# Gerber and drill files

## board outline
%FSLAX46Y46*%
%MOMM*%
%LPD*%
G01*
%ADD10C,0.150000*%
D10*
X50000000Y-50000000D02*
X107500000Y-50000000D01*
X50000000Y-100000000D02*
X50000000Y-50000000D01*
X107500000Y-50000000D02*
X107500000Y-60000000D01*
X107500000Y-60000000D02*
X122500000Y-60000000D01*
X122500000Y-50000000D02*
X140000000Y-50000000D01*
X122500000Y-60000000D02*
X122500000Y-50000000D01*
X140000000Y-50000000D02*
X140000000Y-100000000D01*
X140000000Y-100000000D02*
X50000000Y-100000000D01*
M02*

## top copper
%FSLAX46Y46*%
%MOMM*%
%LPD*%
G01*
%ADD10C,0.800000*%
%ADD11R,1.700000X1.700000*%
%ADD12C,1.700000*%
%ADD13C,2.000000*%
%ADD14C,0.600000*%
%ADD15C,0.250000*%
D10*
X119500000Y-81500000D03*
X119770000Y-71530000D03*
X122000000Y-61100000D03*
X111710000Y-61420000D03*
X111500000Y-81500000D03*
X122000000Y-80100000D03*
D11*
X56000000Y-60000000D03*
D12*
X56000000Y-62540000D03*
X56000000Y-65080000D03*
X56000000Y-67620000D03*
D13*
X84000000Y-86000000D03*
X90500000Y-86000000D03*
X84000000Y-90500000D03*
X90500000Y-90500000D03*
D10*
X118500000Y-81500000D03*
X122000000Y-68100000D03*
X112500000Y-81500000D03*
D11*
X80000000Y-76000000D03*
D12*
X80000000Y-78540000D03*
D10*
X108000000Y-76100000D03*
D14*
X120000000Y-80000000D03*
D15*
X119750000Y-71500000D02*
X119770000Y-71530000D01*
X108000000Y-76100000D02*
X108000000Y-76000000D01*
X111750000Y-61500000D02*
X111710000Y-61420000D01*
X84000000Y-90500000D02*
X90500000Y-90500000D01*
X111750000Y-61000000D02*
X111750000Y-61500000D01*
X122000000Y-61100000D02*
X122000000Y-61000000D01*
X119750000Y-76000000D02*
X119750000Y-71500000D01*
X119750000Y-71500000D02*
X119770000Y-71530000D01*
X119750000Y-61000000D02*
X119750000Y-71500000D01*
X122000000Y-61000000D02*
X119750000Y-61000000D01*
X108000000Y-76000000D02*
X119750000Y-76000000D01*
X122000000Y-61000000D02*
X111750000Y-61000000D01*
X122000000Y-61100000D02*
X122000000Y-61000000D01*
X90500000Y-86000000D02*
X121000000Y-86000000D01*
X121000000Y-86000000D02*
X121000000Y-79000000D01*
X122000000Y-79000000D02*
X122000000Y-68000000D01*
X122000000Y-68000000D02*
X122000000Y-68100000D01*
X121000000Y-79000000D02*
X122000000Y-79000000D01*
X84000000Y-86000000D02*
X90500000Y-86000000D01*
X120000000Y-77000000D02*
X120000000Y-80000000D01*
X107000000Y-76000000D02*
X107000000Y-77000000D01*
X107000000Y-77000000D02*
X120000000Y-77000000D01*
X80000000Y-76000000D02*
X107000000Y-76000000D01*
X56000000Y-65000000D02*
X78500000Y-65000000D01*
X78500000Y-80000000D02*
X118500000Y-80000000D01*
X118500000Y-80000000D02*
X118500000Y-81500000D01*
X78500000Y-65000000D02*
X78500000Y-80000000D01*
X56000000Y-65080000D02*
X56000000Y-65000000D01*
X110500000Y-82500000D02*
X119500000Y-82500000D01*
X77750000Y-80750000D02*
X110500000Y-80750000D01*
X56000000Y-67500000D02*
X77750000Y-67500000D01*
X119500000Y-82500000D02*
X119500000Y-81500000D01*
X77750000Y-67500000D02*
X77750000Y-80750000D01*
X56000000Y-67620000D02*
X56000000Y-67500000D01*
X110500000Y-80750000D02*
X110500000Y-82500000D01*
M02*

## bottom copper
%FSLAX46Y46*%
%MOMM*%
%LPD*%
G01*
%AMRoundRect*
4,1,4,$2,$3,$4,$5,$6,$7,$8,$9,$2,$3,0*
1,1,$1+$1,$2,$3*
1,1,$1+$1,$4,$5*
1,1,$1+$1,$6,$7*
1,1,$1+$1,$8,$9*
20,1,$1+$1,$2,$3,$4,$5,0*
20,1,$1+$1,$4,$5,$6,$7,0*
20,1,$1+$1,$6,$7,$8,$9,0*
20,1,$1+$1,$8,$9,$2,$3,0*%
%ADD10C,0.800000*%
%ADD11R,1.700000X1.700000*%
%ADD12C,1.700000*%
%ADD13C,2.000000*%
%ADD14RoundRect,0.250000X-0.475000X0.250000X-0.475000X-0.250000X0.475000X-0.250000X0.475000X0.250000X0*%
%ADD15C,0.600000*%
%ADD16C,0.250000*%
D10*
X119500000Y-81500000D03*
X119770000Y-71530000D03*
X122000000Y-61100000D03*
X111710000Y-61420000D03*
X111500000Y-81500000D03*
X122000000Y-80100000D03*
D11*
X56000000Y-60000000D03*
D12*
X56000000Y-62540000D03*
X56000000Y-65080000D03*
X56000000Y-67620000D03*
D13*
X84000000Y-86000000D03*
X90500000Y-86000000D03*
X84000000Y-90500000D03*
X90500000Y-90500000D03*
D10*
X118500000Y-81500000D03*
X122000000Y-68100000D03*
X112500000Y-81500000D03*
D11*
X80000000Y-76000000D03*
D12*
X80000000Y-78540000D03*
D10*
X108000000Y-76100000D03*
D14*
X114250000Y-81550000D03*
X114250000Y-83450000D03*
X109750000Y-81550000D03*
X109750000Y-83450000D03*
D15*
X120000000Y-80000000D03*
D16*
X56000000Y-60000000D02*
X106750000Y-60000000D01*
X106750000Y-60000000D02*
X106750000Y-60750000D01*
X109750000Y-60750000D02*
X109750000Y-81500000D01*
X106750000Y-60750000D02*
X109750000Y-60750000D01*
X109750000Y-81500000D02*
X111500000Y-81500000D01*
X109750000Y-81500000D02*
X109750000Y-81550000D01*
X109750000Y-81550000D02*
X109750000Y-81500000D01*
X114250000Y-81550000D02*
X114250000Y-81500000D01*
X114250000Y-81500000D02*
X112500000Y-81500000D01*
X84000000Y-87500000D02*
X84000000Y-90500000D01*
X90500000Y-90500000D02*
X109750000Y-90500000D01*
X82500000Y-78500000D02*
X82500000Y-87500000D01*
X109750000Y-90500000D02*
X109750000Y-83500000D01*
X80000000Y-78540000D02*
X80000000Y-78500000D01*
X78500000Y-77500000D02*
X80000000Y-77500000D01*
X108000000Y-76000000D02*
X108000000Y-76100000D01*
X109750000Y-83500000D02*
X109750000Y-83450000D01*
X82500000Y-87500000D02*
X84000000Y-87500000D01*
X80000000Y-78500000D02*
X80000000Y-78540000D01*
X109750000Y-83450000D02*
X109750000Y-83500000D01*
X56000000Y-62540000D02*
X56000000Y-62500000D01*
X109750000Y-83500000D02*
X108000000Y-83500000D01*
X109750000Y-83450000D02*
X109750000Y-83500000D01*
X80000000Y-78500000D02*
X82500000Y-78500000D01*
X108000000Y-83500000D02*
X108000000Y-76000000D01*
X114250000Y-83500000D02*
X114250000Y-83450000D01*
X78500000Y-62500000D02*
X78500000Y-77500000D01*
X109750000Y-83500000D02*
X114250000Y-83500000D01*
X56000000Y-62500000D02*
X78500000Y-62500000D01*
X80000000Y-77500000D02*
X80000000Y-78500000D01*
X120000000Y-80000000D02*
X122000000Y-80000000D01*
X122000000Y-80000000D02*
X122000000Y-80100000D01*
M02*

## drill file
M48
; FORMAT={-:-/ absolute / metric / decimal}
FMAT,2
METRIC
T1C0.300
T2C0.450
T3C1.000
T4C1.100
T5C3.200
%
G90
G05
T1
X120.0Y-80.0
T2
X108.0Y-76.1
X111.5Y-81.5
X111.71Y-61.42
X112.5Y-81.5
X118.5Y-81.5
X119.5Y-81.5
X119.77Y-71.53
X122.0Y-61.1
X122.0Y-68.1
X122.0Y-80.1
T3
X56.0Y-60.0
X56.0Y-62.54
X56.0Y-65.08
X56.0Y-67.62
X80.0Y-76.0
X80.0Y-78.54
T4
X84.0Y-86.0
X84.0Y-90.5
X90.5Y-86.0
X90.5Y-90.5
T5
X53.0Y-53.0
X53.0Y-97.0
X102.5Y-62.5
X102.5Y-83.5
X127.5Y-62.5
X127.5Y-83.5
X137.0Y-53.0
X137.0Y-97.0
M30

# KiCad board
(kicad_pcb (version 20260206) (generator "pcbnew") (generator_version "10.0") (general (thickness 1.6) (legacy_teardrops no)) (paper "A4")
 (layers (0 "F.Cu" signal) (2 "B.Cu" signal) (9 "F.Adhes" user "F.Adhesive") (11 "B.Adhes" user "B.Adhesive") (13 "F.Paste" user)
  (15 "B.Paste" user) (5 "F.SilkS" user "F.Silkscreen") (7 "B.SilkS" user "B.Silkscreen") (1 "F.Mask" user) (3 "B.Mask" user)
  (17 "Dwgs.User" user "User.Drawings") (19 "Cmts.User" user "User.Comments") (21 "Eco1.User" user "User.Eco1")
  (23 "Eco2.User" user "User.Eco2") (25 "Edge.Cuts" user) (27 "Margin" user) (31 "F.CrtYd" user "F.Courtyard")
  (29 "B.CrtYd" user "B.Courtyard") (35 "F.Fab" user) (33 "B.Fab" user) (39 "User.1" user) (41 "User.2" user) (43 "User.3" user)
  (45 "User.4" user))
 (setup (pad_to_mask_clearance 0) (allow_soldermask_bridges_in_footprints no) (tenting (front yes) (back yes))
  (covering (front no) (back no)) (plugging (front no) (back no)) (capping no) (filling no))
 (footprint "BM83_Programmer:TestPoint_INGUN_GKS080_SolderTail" (layer "F.Cu") (at 119.5 81.5)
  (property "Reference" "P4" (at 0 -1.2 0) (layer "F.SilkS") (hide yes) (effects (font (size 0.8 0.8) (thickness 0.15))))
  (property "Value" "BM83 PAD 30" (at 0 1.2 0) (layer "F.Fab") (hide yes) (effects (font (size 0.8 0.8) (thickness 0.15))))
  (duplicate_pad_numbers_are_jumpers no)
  (pad "1" thru_hole circle (at 0 0) (size 0.8 0.8) (drill 0.45) (layers "*.Cu" "*.Mask") (remove_unused_layers no) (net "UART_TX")))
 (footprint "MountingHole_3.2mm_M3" (layer "F.Cu") (at 53 97)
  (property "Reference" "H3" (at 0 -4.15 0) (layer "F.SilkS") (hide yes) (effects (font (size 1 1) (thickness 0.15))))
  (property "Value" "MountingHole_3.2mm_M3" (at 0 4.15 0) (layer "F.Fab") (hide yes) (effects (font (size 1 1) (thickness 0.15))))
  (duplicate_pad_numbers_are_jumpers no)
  (pad "" np_thru_hole circle (at 0 0) (size 3.2 3.2) (drill 3.2) (layers "*.Cu" "*.Mask")))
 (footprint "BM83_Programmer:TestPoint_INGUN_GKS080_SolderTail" (layer "F.Cu") (at 119.77 71.53)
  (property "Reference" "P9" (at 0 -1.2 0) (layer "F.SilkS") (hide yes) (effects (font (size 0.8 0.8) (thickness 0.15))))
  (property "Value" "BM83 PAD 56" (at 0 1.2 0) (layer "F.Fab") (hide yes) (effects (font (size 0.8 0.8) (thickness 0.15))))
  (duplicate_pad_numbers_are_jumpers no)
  (pad "1" thru_hole circle (at 0 0) (size 0.8 0.8) (drill 0.45) (layers "*.Cu" "*.Mask") (remove_unused_layers no) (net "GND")))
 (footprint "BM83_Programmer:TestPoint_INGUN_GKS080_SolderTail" (layer "F.Cu") (at 122 61.1)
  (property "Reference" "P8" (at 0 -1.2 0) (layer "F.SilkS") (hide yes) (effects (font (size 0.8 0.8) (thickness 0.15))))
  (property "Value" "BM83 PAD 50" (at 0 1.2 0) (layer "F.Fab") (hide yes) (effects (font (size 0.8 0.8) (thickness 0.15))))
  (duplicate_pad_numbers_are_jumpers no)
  (pad "1" thru_hole circle (at 0 0) (size 0.8 0.8) (drill 0.45) (layers "*.Cu" "*.Mask") (remove_unused_layers no) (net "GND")))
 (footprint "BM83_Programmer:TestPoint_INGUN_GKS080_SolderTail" (layer "F.Cu") (at 111.71 61.42)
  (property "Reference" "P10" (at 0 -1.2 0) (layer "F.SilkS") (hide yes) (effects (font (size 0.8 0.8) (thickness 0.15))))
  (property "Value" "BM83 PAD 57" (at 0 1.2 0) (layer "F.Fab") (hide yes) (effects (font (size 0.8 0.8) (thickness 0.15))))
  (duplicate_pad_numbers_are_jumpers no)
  (pad "1" thru_hole circle (at 0 0) (size 0.8 0.8) (drill 0.45) (layers "*.Cu" "*.Mask") (remove_unused_layers no) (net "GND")))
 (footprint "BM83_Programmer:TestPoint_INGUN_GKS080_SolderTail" (layer "F.Cu") (at 111.5 81.5)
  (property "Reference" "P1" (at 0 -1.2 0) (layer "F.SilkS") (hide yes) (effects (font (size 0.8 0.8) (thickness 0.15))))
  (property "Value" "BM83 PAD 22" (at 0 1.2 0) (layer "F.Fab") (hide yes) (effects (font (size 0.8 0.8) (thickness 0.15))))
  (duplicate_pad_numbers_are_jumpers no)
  (pad "1" thru_hole circle (at 0 0) (size 0.8 0.8) (drill 0.45) (layers "*.Cu" "*.Mask") (remove_unused_layers no) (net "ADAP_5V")))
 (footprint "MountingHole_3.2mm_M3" (layer "F.Cu") (at 102.5 62.5)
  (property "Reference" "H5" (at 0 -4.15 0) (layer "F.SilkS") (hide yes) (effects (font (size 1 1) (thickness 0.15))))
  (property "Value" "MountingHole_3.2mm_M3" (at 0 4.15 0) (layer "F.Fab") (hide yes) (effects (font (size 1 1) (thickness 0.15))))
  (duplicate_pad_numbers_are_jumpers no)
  (pad "" np_thru_hole circle (at 0 0) (size 3.2 3.2) (drill 3.2) (layers "*.Cu" "*.Mask")))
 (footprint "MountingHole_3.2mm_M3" (layer "F.Cu") (at 127.5 83.5)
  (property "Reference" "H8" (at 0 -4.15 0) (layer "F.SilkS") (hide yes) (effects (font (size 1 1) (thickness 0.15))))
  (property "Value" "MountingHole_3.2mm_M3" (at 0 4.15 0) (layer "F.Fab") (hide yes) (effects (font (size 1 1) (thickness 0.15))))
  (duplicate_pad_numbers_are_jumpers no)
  (pad "" np_thru_hole circle (at 0 0) (size 3.2 3.2) (drill 3.2) (layers "*.Cu" "*.Mask")))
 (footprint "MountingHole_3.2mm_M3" (layer "F.Cu") (at 53 53)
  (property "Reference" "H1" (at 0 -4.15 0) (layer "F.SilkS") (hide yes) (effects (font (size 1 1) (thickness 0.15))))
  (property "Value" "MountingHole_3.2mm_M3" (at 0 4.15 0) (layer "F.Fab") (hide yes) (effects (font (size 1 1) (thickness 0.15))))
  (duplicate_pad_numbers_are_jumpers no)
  (pad "" np_thru_hole circle (at 0 0) (size 3.2 3.2) (drill 3.2) (layers "*.Cu" "*.Mask")))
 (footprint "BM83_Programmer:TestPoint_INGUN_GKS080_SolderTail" (layer "F.Cu") (at 122 80.1)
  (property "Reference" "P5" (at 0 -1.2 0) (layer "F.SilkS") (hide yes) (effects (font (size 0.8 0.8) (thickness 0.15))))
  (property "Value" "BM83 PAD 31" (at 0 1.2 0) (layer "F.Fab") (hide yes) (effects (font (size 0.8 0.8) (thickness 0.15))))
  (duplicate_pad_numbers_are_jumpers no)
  (pad "1" thru_hole circle (at 0 0) (size 0.8 0.8) (drill 0.45) (layers "*.Cu" "*.Mask") (remove_unused_layers no) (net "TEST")))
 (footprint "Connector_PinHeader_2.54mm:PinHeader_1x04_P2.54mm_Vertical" (layer "F.Cu") (at 56 60)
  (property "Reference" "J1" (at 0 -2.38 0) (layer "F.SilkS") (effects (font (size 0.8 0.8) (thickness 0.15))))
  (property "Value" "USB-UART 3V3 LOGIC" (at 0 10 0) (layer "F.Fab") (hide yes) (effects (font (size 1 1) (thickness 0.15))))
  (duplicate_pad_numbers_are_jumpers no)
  (pad "1" thru_hole rect (at 0 0) (size 1.7 1.7) (drill 1) (layers "*.Cu" "*.Mask") (remove_unused_layers no) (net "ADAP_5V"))
  (pad "2" thru_hole circle (at 0 2.54) (size 1.7 1.7) (drill 1) (layers "*.Cu" "*.Mask") (remove_unused_layers no) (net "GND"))
  (pad "3" thru_hole circle (at 0 5.08) (size 1.7 1.7) (drill 1) (layers "*.Cu" "*.Mask") (remove_unused_layers no) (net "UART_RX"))
  (pad "4" thru_hole circle (at 0 7.62) (size 1.7 1.7) (drill 1) (layers "*.Cu" "*.Mask") (remove_unused_layers no) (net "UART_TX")))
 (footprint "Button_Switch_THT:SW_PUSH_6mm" (layer "F.Cu") (at 84 86)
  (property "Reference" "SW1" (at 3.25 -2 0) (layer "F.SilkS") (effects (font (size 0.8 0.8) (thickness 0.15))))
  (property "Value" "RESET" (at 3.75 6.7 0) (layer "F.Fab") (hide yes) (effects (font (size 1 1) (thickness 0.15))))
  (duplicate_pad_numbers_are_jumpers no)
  (pad "1" thru_hole circle (at 0 0 90) (size 2 2) (drill 1.1) (layers "*.Cu" "*.Mask") (remove_unused_layers no) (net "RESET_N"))
  (pad "1" thru_hole circle (at 6.5 0 90) (size 2 2) (drill 1.1) (layers "*.Cu" "*.Mask") (remove_unused_layers no) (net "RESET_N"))
  (pad "2" thru_hole circle (at 0 4.5 90) (size 2 2) (drill 1.1) (layers "*.Cu" "*.Mask") (remove_unused_layers no) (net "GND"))
  (pad "2" thru_hole circle (at 6.5 4.5 90) (size 2 2) (drill 1.1) (layers "*.Cu" "*.Mask") (remove_unused_layers no) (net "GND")))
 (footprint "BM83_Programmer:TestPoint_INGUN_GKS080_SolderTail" (layer "F.Cu") (at 118.5 81.5)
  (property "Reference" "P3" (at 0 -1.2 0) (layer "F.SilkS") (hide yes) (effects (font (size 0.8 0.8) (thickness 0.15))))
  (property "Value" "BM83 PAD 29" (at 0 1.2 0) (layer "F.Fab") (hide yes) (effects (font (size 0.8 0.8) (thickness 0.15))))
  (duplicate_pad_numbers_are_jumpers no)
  (pad "1" thru_hole circle (at 0 0) (size 0.8 0.8) (drill 0.45) (layers "*.Cu" "*.Mask") (remove_unused_layers no) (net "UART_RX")))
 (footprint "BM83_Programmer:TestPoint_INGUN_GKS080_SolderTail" (layer "F.Cu") (at 122 68.1)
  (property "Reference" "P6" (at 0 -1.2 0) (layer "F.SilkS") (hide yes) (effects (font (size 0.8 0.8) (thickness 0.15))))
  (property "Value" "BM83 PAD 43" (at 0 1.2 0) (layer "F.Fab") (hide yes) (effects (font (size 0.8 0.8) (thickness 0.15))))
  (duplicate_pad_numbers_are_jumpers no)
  (pad "1" thru_hole circle (at 0 0) (size 0.8 0.8) (drill 0.45) (layers "*.Cu" "*.Mask") (remove_unused_layers no) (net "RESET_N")))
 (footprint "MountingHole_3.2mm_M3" (layer "F.Cu") (at 127.5 62.5)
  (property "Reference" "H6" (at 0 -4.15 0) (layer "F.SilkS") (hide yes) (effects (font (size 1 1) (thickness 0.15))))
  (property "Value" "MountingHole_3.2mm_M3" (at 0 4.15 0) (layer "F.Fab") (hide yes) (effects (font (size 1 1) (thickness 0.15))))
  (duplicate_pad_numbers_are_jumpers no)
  (pad "" np_thru_hole circle (at 0 0) (size 3.2 3.2) (drill 3.2) (layers "*.Cu" "*.Mask")))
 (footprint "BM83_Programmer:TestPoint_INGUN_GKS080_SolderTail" (layer "F.Cu") (at 112.5 81.5)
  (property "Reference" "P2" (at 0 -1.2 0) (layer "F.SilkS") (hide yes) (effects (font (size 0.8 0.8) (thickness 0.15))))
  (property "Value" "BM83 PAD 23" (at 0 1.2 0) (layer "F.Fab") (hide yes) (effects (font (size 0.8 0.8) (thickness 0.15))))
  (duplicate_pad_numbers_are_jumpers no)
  (pad "1" thru_hole circle (at 0 0) (size 0.8 0.8) (drill 0.45) (layers "*.Cu" "*.Mask") (remove_unused_layers no) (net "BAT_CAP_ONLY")))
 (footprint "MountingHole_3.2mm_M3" (layer "F.Cu") (at 137 53)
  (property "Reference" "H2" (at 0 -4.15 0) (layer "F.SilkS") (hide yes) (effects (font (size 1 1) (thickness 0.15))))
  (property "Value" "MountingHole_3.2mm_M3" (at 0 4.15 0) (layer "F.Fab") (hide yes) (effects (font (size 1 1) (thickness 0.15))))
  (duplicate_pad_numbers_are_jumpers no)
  (pad "" np_thru_hole circle (at 0 0) (size 3.2 3.2) (drill 3.2) (layers "*.Cu" "*.Mask")))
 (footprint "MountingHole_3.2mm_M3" (layer "F.Cu") (at 137 97)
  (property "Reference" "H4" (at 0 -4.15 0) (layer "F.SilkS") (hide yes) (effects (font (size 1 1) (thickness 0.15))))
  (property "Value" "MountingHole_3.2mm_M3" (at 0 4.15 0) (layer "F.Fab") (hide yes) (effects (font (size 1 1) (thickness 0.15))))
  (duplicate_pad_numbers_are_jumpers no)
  (pad "" np_thru_hole circle (at 0 0) (size 3.2 3.2) (drill 3.2) (layers "*.Cu" "*.Mask")))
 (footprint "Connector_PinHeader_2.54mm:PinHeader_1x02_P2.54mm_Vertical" (layer "F.Cu") (at 80 76)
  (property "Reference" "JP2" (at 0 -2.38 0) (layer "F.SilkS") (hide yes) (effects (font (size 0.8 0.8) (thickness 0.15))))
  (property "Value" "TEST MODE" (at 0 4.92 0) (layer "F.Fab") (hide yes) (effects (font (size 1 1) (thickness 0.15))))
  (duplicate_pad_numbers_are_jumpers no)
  (pad "1" thru_hole rect (at 0 0) (size 1.7 1.7) (drill 1) (layers "*.Cu" "*.Mask") (remove_unused_layers no) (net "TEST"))
  (pad "2" thru_hole circle (at 0 2.54) (size 1.7 1.7) (drill 1) (layers "*.Cu" "*.Mask") (remove_unused_layers no) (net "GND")))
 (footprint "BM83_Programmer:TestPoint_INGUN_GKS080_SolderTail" (layer "F.Cu") (at 108 76.1)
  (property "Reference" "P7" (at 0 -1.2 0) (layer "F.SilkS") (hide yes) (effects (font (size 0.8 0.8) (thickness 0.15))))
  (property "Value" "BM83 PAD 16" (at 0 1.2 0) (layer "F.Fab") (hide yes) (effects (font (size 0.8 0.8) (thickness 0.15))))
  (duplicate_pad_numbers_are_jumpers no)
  (pad "1" thru_hole circle (at 0 0) (size 0.8 0.8) (drill 0.45) (layers "*.Cu" "*.Mask") (remove_unused_layers no) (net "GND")))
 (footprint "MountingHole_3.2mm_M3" (layer "F.Cu") (at 102.5 83.5)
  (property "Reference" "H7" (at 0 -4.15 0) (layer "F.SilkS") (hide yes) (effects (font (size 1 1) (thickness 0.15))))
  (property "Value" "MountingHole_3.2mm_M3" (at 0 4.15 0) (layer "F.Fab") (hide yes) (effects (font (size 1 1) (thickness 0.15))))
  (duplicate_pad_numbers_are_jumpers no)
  (pad "" np_thru_hole circle (at 0 0) (size 3.2 3.2) (drill 3.2) (layers "*.Cu" "*.Mask")))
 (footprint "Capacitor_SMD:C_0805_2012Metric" (layer "B.Cu") (at 114.25 82.5 -90)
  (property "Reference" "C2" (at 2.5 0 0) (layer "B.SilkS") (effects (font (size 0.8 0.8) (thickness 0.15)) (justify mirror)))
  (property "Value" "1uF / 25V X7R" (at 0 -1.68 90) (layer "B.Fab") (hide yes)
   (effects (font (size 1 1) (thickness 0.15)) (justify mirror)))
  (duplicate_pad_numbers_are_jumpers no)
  (pad "1" smd roundrect (at -0.95 0 270) (size 1 1.45) (layers "B.Cu" "B.Mask" "B.Paste") (roundrect_rratio 0.25) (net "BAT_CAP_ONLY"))
  (pad "2" smd roundrect (at 0.95 0 270) (size 1 1.45) (layers "B.Cu" "B.Mask" "B.Paste") (roundrect_rratio 0.25) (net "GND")))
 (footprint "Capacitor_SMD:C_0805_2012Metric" (layer "B.Cu") (at 109.75 82.5 -90)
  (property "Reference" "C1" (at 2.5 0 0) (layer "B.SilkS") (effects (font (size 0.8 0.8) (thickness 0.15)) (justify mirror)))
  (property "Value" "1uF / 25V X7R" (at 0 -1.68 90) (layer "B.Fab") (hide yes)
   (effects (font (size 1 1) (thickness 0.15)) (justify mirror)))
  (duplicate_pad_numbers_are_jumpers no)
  (pad "1" smd roundrect (at -0.95 0 270) (size 1 1.45) (layers "B.Cu" "B.Mask" "B.Paste") (roundrect_rratio 0.25) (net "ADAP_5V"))
  (pad "2" smd roundrect (at 0.95 0 270) (size 1 1.45) (layers "B.Cu" "B.Mask" "B.Paste") (roundrect_rratio 0.25) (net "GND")))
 (gr_line (start 50 50) (end 107.5 50) (stroke (width 0.15) (type default)) (layer "Edge.Cuts"))
 (gr_line (start 50 100) (end 50 50) (stroke (width 0.15) (type default)) (layer "Edge.Cuts"))
 (gr_line (start 107.5 50) (end 107.5 60) (stroke (width 0.15) (type default)) (layer "Edge.Cuts"))
 (gr_line (start 107.5 60) (end 122.5 60) (stroke (width 0.15) (type default)) (layer "Edge.Cuts"))
 (gr_line (start 122.5 50) (end 140 50) (stroke (width 0.15) (type default)) (layer "Edge.Cuts"))
 (gr_line (start 122.5 60) (end 122.5 50) (stroke (width 0.15) (type default)) (layer "Edge.Cuts"))
 (gr_line (start 140 50) (end 140 100) (stroke (width 0.15) (type default)) (layer "Edge.Cuts"))
 (gr_line (start 140 100) (end 50 100) (stroke (width 0.15) (type default)) (layer "Edge.Cuts"))
 (segment (start 56 60) (end 106.75 60) (width 0.25) (layer "B.Cu") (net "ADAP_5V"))
 (segment (start 106.75 60) (end 106.75 60.75) (width 0.25) (layer "B.Cu") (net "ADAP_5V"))
 (segment (start 109.75 60.75) (end 109.75 81.5) (width 0.25) (layer "B.Cu") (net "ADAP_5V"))
 (segment (start 106.75 60.75) (end 109.75 60.75) (width 0.25) (layer "B.Cu") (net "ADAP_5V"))
 (segment (start 109.75 81.5) (end 111.5 81.5) (width 0.25) (layer "B.Cu") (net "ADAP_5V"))
 (segment (start 109.75 81.5) (end 109.75 81.55) (width 0.25) (layer "B.Cu") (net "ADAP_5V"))
 (segment (start 109.75 81.55) (end 109.75 81.5) (width 0.25) (layer "B.Cu") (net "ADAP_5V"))
 (segment (start 114.25 81.55) (end 114.25 81.5) (width 0.25) (layer "B.Cu") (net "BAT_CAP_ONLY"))
 (segment (start 114.25 81.5) (end 112.5 81.5) (width 0.25) (layer "B.Cu") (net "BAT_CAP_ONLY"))
 (segment (start 119.75 71.5) (end 119.77 71.53) (width 0.25) (layer "F.Cu") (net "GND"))
 (segment (start 108 76.1) (end 108 76) (width 0.25) (layer "F.Cu") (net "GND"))
 (segment (start 111.75 61.5) (end 111.71 61.42) (width 0.25) (layer "F.Cu") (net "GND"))
 (segment (start 84 90.5) (end 90.5 90.5) (width 0.25) (layer "F.Cu") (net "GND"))
 (segment (start 111.75 61) (end 111.75 61.5) (width 0.25) (layer "F.Cu") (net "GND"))
 (segment (start 122 61.1) (end 122 61) (width 0.25) (layer "F.Cu") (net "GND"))
 (segment (start 119.75 76) (end 119.75 71.5) (width 0.25) (layer "F.Cu") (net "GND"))
 (segment (start 119.75 71.5) (end 119.77 71.53) (width 0.25) (layer "F.Cu") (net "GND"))
 (segment (start 119.75 61) (end 119.75 71.5) (width 0.25) (layer "F.Cu") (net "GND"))
 (segment (start 122 61) (end 119.75 61) (width 0.25) (layer "F.Cu") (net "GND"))
 (segment (start 108 76) (end 119.75 76) (width 0.25) (layer "F.Cu") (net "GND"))
 (segment (start 122 61) (end 111.75 61) (width 0.25) (layer "F.Cu") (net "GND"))
 (segment (start 122 61.1) (end 122 61) (width 0.25) (layer "F.Cu") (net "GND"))
 (segment (start 84 87.5) (end 84 90.5) (width 0.25) (layer "B.Cu") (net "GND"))
 (segment (start 90.5 90.5) (end 109.75 90.5) (width 0.25) (layer "B.Cu") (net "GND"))
 (segment (start 82.5 78.5) (end 82.5 87.5) (width 0.25) (layer "B.Cu") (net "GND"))
 (segment (start 109.75 90.5) (end 109.75 83.5) (width 0.25) (layer "B.Cu") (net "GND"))
 (segment (start 80 78.54) (end 80 78.5) (width 0.25) (layer "B.Cu") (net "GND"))
 (segment (start 78.5 77.5) (end 80 77.5) (width 0.25) (layer "B.Cu") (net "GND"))
 (segment (start 108 76) (end 108 76.1) (width 0.25) (layer "B.Cu") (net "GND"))
 (segment (start 109.75 83.5) (end 109.75 83.45) (width 0.25) (layer "B.Cu") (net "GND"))
 (segment (start 82.5 87.5) (end 84 87.5) (width 0.25) (layer "B.Cu") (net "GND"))
 (segment (start 80 78.5) (end 80 78.54) (width 0.25) (layer "B.Cu") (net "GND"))
 (segment (start 109.75 83.45) (end 109.75 83.5) (width 0.25) (layer "B.Cu") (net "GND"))
 (segment (start 56 62.54) (end 56 62.5) (width 0.25) (layer "B.Cu") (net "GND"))
 (segment (start 109.75 83.5) (end 108 83.5) (width 0.25) (layer "B.Cu") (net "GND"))
 (segment (start 109.75 83.45) (end 109.75 83.5) (width 0.25) (layer "B.Cu") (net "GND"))
 (segment (start 80 78.5) (end 82.5 78.5) (width 0.25) (layer "B.Cu") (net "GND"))
 (segment (start 108 83.5) (end 108 76) (width 0.25) (layer "B.Cu") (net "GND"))
 (segment (start 114.25 83.5) (end 114.25 83.45) (width 0.25) (layer "B.Cu") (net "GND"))
 (segment (start 78.5 62.5) (end 78.5 77.5) (width 0.25) (layer "B.Cu") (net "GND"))
 (segment (start 109.75 83.5) (end 114.25 83.5) (width 0.25) (layer "B.Cu") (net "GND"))
 (segment (start 56 62.5) (end 78.5 62.5) (width 0.25) (layer "B.Cu") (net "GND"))
 (segment (start 80 77.5) (end 80 78.5) (width 0.25) (layer "B.Cu") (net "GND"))
 (segment (start 90.5 86) (end 121 86) (width 0.25) (layer "F.Cu") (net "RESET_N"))
 (segment (start 121 86) (end 121 79) (width 0.25) (layer "F.Cu") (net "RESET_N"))
 (segment (start 122 79) (end 122 68) (width 0.25) (layer "F.Cu") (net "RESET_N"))
 (segment (start 122 68) (end 122 68.1) (width 0.25) (layer "F.Cu") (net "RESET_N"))
 (segment (start 121 79) (end 122 79) (width 0.25) (layer "F.Cu") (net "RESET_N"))
 (segment (start 84 86) (end 90.5 86) (width 0.25) (layer "F.Cu") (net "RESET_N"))
 (segment (start 120 77) (end 120 80) (width 0.25) (layer "F.Cu") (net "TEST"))
 (segment (start 107 76) (end 107 77) (width 0.25) (layer "F.Cu") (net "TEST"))
 (segment (start 107 77) (end 120 77) (width 0.25) (layer "F.Cu") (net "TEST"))
 (segment (start 80 76) (end 107 76) (width 0.25) (layer "F.Cu") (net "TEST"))
 (via (at 120 80) (size 0.6) (drill 0.3) (layers "F.Cu" "B.Cu") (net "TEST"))
 (segment (start 120 80) (end 122 80) (width 0.25) (layer "B.Cu") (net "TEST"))
 (segment (start 122 80) (end 122 80.1) (width 0.25) (layer "B.Cu") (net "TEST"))
 (segment (start 56 65) (end 78.5 65) (width 0.25) (layer "F.Cu") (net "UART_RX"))
 (segment (start 78.5 80) (end 118.5 80) (width 0.25) (layer "F.Cu") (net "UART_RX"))
 (segment (start 118.5 80) (end 118.5 81.5) (width 0.25) (layer "F.Cu") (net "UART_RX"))
 (segment (start 78.5 65) (end 78.5 80) (width 0.25) (layer "F.Cu") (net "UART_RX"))
 (segment (start 56 65.08) (end 56 65) (width 0.25) (layer "F.Cu") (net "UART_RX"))
 (segment (start 110.5 82.5) (end 119.5 82.5) (width 0.25) (layer "F.Cu") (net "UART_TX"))
 (segment (start 77.75 80.75) (end 110.5 80.75) (width 0.25) (layer "F.Cu") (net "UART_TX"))
 (segment (start 56 67.5) (end 77.75 67.5) (width 0.25) (layer "F.Cu") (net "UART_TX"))
 (segment (start 119.5 82.5) (end 119.5 81.5) (width 0.25) (layer "F.Cu") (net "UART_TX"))
 (segment (start 77.75 67.5) (end 77.75 80.75) (width 0.25) (layer "F.Cu") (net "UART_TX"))
 (segment (start 56 67.62) (end 56 67.5) (width 0.25) (layer "F.Cu") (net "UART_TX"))
 (segment (start 110.5 80.75) (end 110.5 82.5) (width 0.25) (layer "F.Cu") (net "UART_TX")))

